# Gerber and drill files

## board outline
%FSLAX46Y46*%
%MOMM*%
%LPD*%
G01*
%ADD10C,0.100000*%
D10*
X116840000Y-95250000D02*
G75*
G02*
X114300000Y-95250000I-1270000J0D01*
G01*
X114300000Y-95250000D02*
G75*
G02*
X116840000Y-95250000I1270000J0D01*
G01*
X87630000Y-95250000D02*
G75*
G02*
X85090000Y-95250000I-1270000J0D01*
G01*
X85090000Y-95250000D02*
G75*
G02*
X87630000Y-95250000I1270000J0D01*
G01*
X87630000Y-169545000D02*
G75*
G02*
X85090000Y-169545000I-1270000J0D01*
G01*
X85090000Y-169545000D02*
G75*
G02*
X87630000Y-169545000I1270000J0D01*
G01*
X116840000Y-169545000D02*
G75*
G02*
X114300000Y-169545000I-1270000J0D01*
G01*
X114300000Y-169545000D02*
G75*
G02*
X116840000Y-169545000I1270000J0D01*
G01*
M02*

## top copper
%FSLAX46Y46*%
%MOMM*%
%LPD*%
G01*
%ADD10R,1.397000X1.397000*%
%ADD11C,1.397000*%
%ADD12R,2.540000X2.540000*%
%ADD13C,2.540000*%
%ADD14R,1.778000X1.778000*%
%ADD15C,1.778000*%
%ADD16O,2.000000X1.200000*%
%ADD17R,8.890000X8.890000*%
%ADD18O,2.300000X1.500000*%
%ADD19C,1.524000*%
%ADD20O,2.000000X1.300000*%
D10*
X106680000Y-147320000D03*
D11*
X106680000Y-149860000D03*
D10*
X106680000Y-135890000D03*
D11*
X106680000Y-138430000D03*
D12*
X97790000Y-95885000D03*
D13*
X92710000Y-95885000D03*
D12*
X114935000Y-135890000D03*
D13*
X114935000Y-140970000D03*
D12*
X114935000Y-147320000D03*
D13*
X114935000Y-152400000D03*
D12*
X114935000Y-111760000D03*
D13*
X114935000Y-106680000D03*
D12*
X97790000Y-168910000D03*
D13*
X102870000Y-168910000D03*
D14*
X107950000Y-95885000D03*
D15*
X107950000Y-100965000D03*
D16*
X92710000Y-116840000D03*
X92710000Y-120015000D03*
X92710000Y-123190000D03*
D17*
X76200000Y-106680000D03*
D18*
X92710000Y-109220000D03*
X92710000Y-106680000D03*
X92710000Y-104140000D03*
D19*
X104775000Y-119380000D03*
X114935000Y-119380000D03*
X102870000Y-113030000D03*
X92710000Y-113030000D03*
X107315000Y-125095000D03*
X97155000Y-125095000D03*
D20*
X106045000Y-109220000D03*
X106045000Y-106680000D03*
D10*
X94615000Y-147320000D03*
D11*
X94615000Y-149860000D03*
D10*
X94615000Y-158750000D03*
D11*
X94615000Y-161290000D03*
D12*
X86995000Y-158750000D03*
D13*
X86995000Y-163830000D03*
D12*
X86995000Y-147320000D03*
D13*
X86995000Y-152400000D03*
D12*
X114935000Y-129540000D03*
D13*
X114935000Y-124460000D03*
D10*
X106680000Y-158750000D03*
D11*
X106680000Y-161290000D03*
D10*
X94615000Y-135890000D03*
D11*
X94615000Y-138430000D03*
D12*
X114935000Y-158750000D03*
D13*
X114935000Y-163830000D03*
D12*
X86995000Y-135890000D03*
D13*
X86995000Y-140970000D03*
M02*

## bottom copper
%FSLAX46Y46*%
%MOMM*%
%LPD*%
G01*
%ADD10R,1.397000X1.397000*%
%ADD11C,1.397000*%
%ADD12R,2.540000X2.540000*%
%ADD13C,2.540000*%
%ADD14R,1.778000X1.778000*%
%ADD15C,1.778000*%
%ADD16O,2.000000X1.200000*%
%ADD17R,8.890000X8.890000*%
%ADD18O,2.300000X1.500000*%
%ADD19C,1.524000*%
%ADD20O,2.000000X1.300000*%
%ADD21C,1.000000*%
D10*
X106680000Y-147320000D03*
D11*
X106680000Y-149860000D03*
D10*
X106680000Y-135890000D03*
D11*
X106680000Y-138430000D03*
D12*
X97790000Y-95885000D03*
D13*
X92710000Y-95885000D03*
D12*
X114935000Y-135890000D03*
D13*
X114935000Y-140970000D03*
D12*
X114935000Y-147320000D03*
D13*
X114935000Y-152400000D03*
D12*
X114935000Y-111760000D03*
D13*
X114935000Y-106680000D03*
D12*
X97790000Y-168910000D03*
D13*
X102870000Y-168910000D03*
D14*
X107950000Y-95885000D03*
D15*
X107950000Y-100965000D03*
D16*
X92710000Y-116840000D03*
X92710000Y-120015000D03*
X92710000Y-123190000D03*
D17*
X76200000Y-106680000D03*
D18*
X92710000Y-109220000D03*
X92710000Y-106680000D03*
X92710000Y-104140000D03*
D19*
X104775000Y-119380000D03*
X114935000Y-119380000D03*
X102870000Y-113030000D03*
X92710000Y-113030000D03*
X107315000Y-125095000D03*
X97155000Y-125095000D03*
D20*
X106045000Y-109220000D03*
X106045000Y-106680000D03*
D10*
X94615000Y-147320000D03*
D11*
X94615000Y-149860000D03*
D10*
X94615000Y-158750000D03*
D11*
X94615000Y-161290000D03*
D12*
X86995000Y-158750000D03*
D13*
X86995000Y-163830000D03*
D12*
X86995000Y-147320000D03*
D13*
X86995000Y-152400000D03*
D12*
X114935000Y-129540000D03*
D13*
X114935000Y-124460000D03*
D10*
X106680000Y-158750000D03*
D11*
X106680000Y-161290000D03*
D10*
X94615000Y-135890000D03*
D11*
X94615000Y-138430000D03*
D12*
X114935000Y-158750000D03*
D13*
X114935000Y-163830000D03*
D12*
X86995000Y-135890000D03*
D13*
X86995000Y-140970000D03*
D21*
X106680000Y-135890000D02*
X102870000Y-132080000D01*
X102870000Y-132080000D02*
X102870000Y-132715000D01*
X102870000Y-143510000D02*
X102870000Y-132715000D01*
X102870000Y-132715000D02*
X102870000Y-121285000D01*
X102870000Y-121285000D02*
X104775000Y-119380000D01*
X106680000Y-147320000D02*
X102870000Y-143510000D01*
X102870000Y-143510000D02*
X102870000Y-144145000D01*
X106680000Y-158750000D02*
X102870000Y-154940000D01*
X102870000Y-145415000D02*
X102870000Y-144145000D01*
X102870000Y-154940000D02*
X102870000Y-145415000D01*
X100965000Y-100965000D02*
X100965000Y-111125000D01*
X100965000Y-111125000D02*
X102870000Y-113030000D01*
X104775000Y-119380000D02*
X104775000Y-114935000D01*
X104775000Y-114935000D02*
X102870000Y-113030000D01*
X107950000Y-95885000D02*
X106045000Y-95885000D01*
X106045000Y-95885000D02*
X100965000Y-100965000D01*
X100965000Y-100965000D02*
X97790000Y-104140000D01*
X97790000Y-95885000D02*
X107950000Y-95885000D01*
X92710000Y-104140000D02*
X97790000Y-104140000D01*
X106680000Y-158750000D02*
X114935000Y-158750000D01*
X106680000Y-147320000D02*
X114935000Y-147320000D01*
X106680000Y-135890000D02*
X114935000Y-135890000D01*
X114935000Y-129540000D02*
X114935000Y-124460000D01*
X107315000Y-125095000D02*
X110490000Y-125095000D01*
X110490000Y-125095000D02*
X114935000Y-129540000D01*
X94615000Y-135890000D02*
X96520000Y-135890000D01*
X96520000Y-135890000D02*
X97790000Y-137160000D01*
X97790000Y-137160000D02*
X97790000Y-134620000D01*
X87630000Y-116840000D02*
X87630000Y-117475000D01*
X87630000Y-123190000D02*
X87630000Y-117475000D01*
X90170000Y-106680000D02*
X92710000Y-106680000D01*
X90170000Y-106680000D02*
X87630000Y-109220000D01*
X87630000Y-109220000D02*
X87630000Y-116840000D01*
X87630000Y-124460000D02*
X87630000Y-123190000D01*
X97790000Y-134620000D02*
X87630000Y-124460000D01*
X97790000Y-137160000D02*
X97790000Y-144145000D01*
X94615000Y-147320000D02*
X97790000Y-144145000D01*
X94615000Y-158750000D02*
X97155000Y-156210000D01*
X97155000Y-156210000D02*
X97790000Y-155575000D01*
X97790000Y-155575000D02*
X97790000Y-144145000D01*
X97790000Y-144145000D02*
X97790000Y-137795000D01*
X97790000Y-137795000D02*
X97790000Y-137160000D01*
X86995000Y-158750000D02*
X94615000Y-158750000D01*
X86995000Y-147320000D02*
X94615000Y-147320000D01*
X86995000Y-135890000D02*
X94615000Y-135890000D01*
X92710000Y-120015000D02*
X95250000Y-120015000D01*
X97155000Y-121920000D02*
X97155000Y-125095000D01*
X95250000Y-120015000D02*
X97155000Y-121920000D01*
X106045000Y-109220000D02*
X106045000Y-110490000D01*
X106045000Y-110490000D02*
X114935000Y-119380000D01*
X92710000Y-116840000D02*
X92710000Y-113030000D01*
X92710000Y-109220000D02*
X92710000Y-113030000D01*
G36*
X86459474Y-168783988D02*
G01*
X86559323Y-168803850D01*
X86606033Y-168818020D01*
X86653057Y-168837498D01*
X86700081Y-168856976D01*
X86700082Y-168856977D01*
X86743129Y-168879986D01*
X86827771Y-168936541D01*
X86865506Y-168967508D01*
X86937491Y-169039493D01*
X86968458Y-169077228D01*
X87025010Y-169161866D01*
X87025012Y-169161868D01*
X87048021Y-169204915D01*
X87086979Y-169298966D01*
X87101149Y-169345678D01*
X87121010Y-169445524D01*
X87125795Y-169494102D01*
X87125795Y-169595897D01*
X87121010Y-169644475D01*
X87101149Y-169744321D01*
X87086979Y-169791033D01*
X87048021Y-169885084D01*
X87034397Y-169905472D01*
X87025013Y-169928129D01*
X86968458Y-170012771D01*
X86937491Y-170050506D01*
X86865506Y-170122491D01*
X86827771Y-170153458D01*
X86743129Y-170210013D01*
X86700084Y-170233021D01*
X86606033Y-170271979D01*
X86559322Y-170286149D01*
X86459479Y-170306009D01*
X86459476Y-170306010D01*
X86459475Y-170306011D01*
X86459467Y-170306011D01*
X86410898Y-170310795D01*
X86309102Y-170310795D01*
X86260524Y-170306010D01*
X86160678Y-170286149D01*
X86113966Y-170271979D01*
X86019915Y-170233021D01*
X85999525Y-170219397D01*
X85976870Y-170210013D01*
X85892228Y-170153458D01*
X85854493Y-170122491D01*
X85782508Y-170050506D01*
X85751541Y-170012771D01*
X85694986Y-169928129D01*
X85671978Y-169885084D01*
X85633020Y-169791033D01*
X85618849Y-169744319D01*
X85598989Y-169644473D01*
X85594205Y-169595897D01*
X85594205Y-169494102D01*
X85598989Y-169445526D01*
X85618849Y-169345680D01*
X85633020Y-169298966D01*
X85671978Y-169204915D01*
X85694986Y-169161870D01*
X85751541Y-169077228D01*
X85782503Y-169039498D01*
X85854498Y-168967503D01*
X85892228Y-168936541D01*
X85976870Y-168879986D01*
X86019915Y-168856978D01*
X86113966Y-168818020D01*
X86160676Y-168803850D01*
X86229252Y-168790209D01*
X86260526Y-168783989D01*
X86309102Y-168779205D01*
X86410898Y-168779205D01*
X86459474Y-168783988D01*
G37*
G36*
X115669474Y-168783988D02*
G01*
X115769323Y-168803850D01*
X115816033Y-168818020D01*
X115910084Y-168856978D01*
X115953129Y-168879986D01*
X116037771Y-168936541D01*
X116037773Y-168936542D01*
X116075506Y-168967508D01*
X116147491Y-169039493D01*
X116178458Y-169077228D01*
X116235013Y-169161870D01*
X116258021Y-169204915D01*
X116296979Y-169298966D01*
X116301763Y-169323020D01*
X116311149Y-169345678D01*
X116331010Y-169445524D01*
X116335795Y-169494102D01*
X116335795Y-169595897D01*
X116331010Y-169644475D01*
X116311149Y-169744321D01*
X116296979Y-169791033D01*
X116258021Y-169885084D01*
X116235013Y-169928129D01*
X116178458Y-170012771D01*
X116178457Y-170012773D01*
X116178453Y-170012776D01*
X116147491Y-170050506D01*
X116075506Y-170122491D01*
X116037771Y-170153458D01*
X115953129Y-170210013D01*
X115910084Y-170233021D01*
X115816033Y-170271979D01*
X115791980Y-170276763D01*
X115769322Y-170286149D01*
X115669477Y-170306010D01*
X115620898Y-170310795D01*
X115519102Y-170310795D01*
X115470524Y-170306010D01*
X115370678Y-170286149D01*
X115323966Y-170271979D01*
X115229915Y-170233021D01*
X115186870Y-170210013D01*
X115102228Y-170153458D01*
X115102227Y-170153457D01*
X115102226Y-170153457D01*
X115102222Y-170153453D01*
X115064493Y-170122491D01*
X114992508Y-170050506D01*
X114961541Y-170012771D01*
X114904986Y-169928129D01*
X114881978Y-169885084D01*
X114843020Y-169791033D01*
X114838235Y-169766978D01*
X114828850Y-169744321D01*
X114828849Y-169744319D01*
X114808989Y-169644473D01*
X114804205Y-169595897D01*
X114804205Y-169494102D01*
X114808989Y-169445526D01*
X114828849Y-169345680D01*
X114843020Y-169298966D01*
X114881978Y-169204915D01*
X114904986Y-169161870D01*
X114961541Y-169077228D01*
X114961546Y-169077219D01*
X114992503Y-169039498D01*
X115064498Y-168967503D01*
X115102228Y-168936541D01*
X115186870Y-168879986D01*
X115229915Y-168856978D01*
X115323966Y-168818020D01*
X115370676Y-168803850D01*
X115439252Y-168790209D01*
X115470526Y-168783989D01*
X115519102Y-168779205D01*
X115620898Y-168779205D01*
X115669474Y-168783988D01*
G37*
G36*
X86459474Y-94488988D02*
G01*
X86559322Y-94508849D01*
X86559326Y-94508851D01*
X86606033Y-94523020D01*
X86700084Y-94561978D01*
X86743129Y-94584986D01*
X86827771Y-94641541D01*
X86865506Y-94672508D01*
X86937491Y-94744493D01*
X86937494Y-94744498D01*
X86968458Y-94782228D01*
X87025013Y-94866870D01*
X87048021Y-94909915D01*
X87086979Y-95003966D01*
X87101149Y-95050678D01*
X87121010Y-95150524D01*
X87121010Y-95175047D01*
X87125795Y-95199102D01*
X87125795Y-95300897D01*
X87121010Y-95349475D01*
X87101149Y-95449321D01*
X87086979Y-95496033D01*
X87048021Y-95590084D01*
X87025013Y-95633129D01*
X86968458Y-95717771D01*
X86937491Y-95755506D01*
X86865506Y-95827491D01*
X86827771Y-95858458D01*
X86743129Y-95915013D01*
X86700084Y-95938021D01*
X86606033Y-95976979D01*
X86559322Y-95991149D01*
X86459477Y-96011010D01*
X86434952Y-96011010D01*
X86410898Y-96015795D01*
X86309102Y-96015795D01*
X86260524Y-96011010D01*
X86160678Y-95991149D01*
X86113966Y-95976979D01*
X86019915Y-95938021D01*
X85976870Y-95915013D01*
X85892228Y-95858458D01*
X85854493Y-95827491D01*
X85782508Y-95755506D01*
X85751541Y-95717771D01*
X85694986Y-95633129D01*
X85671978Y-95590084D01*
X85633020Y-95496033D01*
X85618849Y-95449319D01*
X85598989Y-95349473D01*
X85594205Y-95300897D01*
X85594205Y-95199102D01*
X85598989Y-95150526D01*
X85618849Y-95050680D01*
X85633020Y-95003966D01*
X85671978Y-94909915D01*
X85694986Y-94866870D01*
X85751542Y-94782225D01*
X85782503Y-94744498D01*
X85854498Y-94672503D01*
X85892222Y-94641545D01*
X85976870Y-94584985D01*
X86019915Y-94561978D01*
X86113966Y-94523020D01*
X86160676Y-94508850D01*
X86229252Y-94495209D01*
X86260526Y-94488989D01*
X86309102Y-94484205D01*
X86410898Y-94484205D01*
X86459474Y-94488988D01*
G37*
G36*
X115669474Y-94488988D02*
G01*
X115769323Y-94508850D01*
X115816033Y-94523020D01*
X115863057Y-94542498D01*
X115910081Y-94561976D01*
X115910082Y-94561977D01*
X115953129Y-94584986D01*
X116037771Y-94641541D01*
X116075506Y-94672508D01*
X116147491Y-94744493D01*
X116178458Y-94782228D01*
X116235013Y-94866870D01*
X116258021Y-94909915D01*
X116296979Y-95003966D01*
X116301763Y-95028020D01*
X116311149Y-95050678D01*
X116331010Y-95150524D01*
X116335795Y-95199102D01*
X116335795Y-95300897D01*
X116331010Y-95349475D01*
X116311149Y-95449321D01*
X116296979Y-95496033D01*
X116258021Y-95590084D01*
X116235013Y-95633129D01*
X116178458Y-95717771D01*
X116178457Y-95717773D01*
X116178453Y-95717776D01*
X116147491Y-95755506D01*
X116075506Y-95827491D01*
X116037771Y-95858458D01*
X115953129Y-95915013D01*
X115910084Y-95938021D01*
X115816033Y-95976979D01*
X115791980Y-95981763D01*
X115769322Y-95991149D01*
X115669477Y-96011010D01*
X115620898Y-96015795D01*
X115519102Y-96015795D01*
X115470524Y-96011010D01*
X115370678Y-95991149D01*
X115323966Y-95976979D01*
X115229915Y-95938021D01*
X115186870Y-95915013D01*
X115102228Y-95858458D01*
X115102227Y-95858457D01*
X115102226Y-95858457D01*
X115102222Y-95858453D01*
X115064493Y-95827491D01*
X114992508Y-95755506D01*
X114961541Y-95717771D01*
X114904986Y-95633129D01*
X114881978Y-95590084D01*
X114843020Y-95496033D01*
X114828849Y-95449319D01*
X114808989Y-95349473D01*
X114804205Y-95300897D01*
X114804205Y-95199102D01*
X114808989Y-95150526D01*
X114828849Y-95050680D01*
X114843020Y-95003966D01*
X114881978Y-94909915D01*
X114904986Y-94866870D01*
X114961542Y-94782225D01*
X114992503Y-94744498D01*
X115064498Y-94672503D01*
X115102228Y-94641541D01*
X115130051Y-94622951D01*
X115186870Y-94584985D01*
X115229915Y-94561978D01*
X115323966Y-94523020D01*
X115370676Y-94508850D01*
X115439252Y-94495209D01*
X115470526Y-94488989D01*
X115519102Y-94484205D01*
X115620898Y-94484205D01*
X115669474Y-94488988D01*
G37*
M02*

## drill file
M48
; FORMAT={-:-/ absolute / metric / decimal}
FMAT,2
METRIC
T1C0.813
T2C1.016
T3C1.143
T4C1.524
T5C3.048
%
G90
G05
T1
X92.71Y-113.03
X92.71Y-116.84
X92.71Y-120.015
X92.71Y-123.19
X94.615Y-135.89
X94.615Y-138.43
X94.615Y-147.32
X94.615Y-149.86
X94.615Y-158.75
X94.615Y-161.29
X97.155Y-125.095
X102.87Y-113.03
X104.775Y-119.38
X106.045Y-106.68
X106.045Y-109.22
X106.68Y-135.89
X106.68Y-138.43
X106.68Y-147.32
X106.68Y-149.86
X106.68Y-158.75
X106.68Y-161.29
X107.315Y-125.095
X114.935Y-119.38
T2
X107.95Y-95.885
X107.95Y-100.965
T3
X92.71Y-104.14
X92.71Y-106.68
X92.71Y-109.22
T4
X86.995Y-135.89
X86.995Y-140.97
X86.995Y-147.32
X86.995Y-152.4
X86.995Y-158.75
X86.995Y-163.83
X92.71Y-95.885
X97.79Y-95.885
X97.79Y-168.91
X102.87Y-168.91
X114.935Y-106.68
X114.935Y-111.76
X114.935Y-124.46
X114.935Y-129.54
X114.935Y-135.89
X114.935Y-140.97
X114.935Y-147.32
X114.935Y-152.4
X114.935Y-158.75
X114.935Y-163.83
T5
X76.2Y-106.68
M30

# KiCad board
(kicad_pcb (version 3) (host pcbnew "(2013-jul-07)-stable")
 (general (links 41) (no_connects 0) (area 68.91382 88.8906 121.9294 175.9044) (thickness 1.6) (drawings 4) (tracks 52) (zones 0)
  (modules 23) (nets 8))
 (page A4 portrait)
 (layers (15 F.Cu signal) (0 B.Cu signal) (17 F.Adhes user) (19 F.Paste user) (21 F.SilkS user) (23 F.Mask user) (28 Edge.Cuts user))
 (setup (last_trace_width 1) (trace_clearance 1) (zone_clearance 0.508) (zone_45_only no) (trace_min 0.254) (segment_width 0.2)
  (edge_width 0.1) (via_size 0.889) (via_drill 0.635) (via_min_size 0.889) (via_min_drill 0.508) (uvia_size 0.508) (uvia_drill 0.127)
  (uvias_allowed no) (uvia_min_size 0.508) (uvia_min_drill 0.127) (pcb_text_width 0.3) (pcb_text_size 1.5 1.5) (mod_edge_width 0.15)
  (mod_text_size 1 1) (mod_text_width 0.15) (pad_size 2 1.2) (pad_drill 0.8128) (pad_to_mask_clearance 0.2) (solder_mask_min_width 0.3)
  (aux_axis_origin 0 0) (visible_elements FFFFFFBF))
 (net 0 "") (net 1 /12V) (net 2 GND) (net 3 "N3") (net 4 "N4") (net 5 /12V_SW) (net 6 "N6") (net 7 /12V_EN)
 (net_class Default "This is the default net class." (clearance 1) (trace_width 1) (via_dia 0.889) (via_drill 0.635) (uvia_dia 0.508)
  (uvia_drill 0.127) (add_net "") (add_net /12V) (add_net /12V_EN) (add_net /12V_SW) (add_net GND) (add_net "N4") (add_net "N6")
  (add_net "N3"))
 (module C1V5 (layer F.Cu) (at 106.68 148.59 270)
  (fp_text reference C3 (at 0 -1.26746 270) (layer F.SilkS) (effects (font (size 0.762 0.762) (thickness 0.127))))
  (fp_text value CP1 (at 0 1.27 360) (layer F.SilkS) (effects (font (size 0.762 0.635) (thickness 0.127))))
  (pad 1 thru_hole rect (at -1.27 0 270) (size 1.397 1.397) (drill 0.8128) (layers *.Cu *.Mask F.SilkS) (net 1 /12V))
  (pad 2 thru_hole circle (at 1.27 0 270) (size 1.397 1.397) (drill 0.8128) (layers *.Cu *.Mask F.SilkS) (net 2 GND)))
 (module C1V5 (layer F.Cu) (at 106.68 137.16 270)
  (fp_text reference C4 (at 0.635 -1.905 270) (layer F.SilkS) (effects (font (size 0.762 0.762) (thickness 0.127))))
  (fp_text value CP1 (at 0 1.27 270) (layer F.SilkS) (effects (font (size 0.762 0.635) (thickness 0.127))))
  (pad 1 thru_hole rect (at -1.27 0 270) (size 1.397 1.397) (drill 0.8128) (layers *.Cu *.Mask F.SilkS) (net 1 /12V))
  (pad 2 thru_hole circle (at 1.27 0 270) (size 1.397 1.397) (drill 0.8128) (layers *.Cu *.Mask F.SilkS) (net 2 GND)))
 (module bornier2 (layer F.Cu) (at 95.25 95.885 180)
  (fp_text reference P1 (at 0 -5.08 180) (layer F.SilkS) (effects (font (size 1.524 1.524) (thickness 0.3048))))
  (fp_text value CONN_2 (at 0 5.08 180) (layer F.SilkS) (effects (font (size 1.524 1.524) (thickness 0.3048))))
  (pad 1 thru_hole rect (at -2.54 0 180) (size 2.54 2.54) (drill 1.524) (layers *.Cu *.Mask F.SilkS) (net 1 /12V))
  (pad 2 thru_hole circle (at 2.54 0 180) (size 2.54 2.54) (drill 1.524) (layers *.Cu *.Mask F.SilkS) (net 2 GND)))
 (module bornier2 (layer F.Cu) (at 114.935 138.43 270)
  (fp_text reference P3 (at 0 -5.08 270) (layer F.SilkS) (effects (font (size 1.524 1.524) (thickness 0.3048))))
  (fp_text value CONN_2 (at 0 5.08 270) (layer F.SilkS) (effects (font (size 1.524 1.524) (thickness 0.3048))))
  (pad 1 thru_hole rect (at -2.54 0 270) (size 2.54 2.54) (drill 1.524) (layers *.Cu *.Mask F.SilkS) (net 1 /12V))
  (pad 2 thru_hole circle (at 2.54 0 270) (size 2.54 2.54) (drill 1.524) (layers *.Cu *.Mask F.SilkS) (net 2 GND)))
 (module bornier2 (layer F.Cu) (at 114.935 149.86 270)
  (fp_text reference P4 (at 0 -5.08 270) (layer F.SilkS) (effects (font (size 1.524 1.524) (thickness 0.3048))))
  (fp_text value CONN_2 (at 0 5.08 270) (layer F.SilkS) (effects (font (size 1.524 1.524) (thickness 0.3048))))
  (pad 1 thru_hole rect (at -2.54 0 270) (size 2.54 2.54) (drill 1.524) (layers *.Cu *.Mask F.SilkS) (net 1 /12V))
  (pad 2 thru_hole circle (at 2.54 0 270) (size 2.54 2.54) (drill 1.524) (layers *.Cu *.Mask F.SilkS) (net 2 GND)))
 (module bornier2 (layer F.Cu) (at 114.935 109.22 90)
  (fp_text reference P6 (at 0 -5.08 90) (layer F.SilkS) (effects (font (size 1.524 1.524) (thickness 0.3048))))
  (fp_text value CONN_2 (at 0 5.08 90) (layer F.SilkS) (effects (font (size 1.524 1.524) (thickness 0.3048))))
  (pad 1 thru_hole rect (at -2.54 0 90) (size 2.54 2.54) (drill 1.524) (layers *.Cu *.Mask F.SilkS) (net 2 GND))
  (pad 2 thru_hole circle (at 2.54 0 90) (size 2.54 2.54) (drill 1.524) (layers *.Cu *.Mask F.SilkS) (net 2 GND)))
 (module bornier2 (layer F.Cu) (at 100.33 168.91)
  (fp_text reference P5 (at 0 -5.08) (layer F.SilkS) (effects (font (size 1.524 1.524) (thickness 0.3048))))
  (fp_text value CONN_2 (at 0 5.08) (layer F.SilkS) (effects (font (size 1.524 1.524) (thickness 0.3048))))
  (pad 1 thru_hole rect (at -2.54 0) (size 2.54 2.54) (drill 1.524) (layers *.Cu *.Mask F.SilkS) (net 2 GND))
  (pad 2 thru_hole circle (at 2.54 0) (size 2.54 2.54) (drill 1.524) (layers *.Cu *.Mask F.SilkS) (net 2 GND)))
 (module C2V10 (layer F.Cu) (at 107.95 98.425 270)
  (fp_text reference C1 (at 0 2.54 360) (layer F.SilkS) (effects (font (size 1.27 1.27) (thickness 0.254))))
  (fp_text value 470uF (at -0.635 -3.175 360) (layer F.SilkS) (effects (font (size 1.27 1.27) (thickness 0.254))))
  (pad 1 thru_hole rect (at -2.54 0 270) (size 1.778 1.778) (drill 1.016) (layers *.Cu *.Mask F.SilkS) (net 1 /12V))
  (pad 2 thru_hole circle (at 2.54 0 270) (size 1.778 1.778) (drill 1.016) (layers *.Cu *.Mask F.SilkS) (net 2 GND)))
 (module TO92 (layer F.Cu) (at 92.71 120.015 45)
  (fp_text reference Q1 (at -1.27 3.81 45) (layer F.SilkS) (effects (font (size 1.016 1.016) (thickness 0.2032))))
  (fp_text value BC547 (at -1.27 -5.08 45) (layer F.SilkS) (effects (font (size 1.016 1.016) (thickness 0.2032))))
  (pad 1 thru_hole oval (at 2.245064 -2.245064 180) (size 2 1.2) (drill 0.8128) (layers *.Cu *.Mask F.SilkS) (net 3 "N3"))
  (pad 2 thru_hole oval (at 0 0 180) (size 2 1.2) (drill 0.8128) (layers *.Cu *.Mask F.SilkS) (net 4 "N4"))
  (pad 3 thru_hole oval (at -2.245064 2.245064 180) (size 2 1.2) (drill 0.8128) (layers *.Cu *.Mask F.SilkS) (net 2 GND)))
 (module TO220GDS (layer F.Cu) (at 92.71 106.68 180)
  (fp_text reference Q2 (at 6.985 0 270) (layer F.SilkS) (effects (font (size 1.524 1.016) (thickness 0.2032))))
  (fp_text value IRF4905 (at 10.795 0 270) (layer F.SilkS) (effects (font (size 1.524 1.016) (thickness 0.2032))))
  (pad 4 thru_hole rect (at 16.51 0 180) (size 8.89 8.89) (drill 3.048) (layers *.Cu *.SilkS *.Mask))
  (pad G thru_hole oval (at 0 -2.54 180) (size 2.3 1.5) (drill 1.143) (layers *.Cu *.Mask F.SilkS) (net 3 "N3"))
  (pad D thru_hole oval (at 0 0 180) (size 2.3 1.5) (drill 1.143) (layers *.Cu *.Mask F.SilkS) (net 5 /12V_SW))
  (pad S thru_hole oval (at 0 2.54 180) (size 2.3 1.5) (drill 1.143) (layers *.Cu *.Mask F.SilkS) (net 1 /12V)))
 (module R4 (layer F.Cu) (at 109.855 119.38) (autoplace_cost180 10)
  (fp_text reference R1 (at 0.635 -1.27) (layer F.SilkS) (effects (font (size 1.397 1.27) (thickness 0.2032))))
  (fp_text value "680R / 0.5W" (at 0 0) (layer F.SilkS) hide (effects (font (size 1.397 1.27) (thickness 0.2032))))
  (pad 1 thru_hole circle (at -5.08 0) (size 1.524 1.524) (drill 0.8128) (layers *.Cu *.Mask F.SilkS) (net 1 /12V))
  (pad 2 thru_hole circle (at 5.08 0) (size 1.524 1.524) (drill 0.8128) (layers *.Cu *.Mask F.SilkS) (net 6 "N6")))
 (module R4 (layer F.Cu) (at 97.79 113.03 180) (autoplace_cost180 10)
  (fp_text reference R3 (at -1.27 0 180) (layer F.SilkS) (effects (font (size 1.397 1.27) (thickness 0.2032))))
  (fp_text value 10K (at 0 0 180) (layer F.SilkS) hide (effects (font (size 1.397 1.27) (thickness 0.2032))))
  (pad 1 thru_hole circle (at -5.08 0 180) (size 1.524 1.524) (drill 0.8128) (layers *.Cu *.Mask F.SilkS) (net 1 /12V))
  (pad 2 thru_hole circle (at 5.08 0 180) (size 1.524 1.524) (drill 0.8128) (layers *.Cu *.Mask F.SilkS) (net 3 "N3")))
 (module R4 (layer F.Cu) (at 102.235 125.095 180) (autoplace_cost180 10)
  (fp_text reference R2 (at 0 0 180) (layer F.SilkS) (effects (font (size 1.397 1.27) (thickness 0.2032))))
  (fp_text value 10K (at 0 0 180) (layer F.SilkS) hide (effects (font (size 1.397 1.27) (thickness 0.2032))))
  (pad 1 thru_hole circle (at -5.08 0 180) (size 1.524 1.524) (drill 0.8128) (layers *.Cu *.Mask F.SilkS) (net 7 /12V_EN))
  (pad 2 thru_hole circle (at 5.08 0 180) (size 1.524 1.524) (drill 0.8128) (layers *.Cu *.Mask F.SilkS) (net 4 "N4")))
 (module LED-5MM (layer F.Cu) (at 106.045 107.95 90)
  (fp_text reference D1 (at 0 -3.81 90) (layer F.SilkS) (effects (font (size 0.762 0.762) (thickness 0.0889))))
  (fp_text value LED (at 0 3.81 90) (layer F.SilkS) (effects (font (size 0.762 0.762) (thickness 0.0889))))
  (pad 1 thru_hole oval (at -1.27 0 90) (size 1.3 2) (drill 0.8128) (layers *.Cu *.Mask F.SilkS) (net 6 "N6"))
  (pad 2 thru_hole oval (at 1.27 0 90) (size 1.3 2) (drill 0.8128) (layers *.Cu *.Mask F.SilkS) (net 2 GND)))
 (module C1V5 (layer F.Cu) (at 94.615 148.59 270)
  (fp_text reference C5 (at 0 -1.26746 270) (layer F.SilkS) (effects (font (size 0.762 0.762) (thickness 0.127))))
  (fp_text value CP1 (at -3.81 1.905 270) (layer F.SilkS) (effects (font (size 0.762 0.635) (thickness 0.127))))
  (pad 1 thru_hole rect (at -1.27 0 270) (size 1.397 1.397) (drill 0.8128) (layers *.Cu *.Mask F.SilkS) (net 5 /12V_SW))
  (pad 2 thru_hole circle (at 1.27 0 270) (size 1.397 1.397) (drill 0.8128) (layers *.Cu *.Mask F.SilkS) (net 2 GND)))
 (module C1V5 (layer F.Cu) (at 94.615 160.02 270)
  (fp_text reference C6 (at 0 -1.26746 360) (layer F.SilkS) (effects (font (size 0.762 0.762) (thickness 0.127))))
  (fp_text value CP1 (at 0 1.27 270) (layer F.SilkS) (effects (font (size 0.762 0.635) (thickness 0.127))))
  (pad 1 thru_hole rect (at -1.27 0 270) (size 1.397 1.397) (drill 0.8128) (layers *.Cu *.Mask F.SilkS) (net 5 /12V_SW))
  (pad 2 thru_hole circle (at 1.27 0 270) (size 1.397 1.397) (drill 0.8128) (layers *.Cu *.Mask F.SilkS) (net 2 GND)))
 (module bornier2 (layer F.Cu) (at 86.995 161.29 270)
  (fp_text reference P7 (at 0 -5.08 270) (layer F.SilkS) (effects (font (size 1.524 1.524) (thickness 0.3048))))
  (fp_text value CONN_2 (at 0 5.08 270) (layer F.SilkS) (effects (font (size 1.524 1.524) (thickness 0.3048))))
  (pad 1 thru_hole rect (at -2.54 0 270) (size 2.54 2.54) (drill 1.524) (layers *.Cu *.Mask F.SilkS) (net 5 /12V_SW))
  (pad 2 thru_hole circle (at 2.54 0 270) (size 2.54 2.54) (drill 1.524) (layers *.Cu *.Mask F.SilkS) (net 2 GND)))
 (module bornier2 (layer F.Cu) (at 86.995 149.86 270)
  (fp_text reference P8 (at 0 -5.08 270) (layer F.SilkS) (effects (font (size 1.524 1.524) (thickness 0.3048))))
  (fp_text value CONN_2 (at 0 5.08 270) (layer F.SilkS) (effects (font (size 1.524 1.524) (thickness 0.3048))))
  (pad 1 thru_hole rect (at -2.54 0 270) (size 2.54 2.54) (drill 1.524) (layers *.Cu *.Mask F.SilkS) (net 5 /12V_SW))
  (pad 2 thru_hole circle (at 2.54 0 270) (size 2.54 2.54) (drill 1.524) (layers *.Cu *.Mask F.SilkS) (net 2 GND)))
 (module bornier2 (layer F.Cu) (at 114.935 127 90)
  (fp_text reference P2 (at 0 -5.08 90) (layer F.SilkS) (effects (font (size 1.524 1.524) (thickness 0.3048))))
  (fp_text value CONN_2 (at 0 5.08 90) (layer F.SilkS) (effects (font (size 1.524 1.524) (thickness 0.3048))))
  (pad 1 thru_hole rect (at -2.54 0 90) (size 2.54 2.54) (drill 1.524) (layers *.Cu *.Mask F.SilkS) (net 7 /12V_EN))
  (pad 2 thru_hole circle (at 2.54 0 90) (size 2.54 2.54) (drill 1.524) (layers *.Cu *.Mask F.SilkS) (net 7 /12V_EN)))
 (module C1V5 (layer F.Cu) (at 106.68 160.02 270)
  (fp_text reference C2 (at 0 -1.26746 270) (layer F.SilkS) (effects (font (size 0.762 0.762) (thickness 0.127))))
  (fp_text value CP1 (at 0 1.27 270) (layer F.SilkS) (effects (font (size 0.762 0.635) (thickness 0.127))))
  (pad 1 thru_hole rect (at -1.27 0 270) (size 1.397 1.397) (drill 0.8128) (layers *.Cu *.Mask F.SilkS) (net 1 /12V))
  (pad 2 thru_hole circle (at 1.27 0 270) (size 1.397 1.397) (drill 0.8128) (layers *.Cu *.Mask F.SilkS) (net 2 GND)))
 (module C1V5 (layer F.Cu) (at 94.615 137.16 270)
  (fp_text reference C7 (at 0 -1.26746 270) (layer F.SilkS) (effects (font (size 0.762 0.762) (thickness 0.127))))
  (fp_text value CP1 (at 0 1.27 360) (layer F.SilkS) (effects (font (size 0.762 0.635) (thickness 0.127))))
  (pad 1 thru_hole rect (at -1.27 0 270) (size 1.397 1.397) (drill 0.8128) (layers *.Cu *.Mask F.SilkS) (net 5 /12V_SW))
  (pad 2 thru_hole circle (at 1.27 0 270) (size 1.397 1.397) (drill 0.8128) (layers *.Cu *.Mask F.SilkS) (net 2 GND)))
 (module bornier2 (layer F.Cu) (at 114.935 161.29 270)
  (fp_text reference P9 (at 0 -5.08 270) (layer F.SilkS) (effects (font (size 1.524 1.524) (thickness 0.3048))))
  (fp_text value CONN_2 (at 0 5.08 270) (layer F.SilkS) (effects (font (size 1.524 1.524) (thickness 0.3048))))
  (pad 1 thru_hole rect (at -2.54 0 270) (size 2.54 2.54) (drill 1.524) (layers *.Cu *.Mask F.SilkS) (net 1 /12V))
  (pad 2 thru_hole circle (at 2.54 0 270) (size 2.54 2.54) (drill 1.524) (layers *.Cu *.Mask F.SilkS) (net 2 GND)))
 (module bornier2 (layer F.Cu) (at 86.995 138.43 270)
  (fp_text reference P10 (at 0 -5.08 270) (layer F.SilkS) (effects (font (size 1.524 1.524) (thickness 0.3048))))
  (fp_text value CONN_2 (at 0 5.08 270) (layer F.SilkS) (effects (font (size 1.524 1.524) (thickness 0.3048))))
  (pad 1 thru_hole rect (at -2.54 0 270) (size 2.54 2.54) (drill 1.524) (layers *.Cu *.Mask F.SilkS) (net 5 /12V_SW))
  (pad 2 thru_hole circle (at 2.54 0 270) (size 2.54 2.54) (drill 1.524) (layers *.Cu *.Mask F.SilkS) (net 2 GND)))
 (gr_circle (center 115.57 95.25) (end 116.84 95.25) (layer Edge.Cuts) (width 0.1))
 (gr_circle (center 86.36 95.25) (end 87.63 95.25) (layer Edge.Cuts) (width 0.1))
 (gr_circle (center 86.36 169.545) (end 87.63 169.545) (layer Edge.Cuts) (width 0.1))
 (gr_circle (center 115.57 169.545) (end 114.3 169.545) (layer Edge.Cuts) (width 0.1))
 (segment (start 106.68 135.89) (end 102.87 132.08) (width 1) (layer B.Cu) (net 1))
 (segment (start 102.87 132.08) (end 102.87 132.715) (width 1) (layer B.Cu) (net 1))
 (segment (start 102.87 143.51) (end 102.87 132.715) (width 1) (layer B.Cu) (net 1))
 (segment (start 102.87 132.715) (end 102.87 121.285) (width 1) (layer B.Cu) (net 1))
 (segment (start 102.87 121.285) (end 104.775 119.38) (width 1) (layer B.Cu) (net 1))
 (segment (start 106.68 147.32) (end 102.87 143.51) (width 1) (layer B.Cu) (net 1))
 (segment (start 102.87 143.51) (end 102.87 144.145) (width 1) (layer B.Cu) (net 1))
 (segment (start 106.68 158.75) (end 102.87 154.94) (width 1) (layer B.Cu) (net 1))
 (segment (start 102.87 145.415) (end 102.87 144.145) (width 1) (layer B.Cu) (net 1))
 (segment (start 102.87 154.94) (end 102.87 145.415) (width 1) (layer B.Cu) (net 1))
 (segment (start 100.965 100.965) (end 100.965 111.125) (width 1) (layer B.Cu) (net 1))
 (segment (start 100.965 111.125) (end 102.87 113.03) (width 1) (layer B.Cu) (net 1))
 (segment (start 104.775 119.38) (end 104.775 114.935) (width 1) (layer B.Cu) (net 1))
 (segment (start 104.775 114.935) (end 102.87 113.03) (width 1) (layer B.Cu) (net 1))
 (segment (start 107.95 95.885) (end 106.045 95.885) (width 1) (layer B.Cu) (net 1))
 (segment (start 106.045 95.885) (end 100.965 100.965) (width 1) (layer B.Cu) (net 1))
 (segment (start 100.965 100.965) (end 97.79 104.14) (width 1) (layer B.Cu) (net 1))
 (segment (start 97.79 95.885) (end 107.95 95.885) (width 1) (layer B.Cu) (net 1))
 (segment (start 92.71 104.14) (end 97.79 104.14) (width 1) (layer B.Cu) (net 1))
 (segment (start 106.68 158.75) (end 114.935 158.75) (width 1) (layer B.Cu) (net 1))
 (segment (start 106.68 147.32) (end 114.935 147.32) (width 1) (layer B.Cu) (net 1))
 (segment (start 106.68 135.89) (end 114.935 135.89) (width 1) (layer B.Cu) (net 1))
 (segment (start 114.935 129.54) (end 114.935 124.46) (width 1) (layer B.Cu) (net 7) (status C00000))
 (segment (start 107.315 125.095) (end 110.49 125.095) (width 1) (layer B.Cu) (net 7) (status 400000))
 (segment (start 110.49 125.095) (end 114.935 129.54) (width 1) (layer B.Cu) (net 7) (status 800000))
 (segment (start 94.615 135.89) (end 96.52 135.89) (width 1) (layer B.Cu) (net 5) (status 400000))
 (segment (start 96.52 135.89) (end 97.79 137.16) (width 1) (layer B.Cu) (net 5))
 (segment (start 97.79 137.16) (end 97.79 134.62) (width 1) (layer B.Cu) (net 5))
 (segment (start 87.63 116.84) (end 87.63 117.475) (width 1) (layer B.Cu) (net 5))
 (segment (start 87.63 123.19) (end 87.63 117.475) (width 1) (layer B.Cu) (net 5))
 (segment (start 90.17 106.68) (end 92.71 106.68) (width 1) (layer B.Cu) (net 5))
 (segment (start 90.17 106.68) (end 87.63 109.22) (width 1) (layer B.Cu) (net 5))
 (segment (start 87.63 109.22) (end 87.63 116.84) (width 1) (layer B.Cu) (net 5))
 (segment (start 87.63 124.46) (end 87.63 123.19) (width 1) (layer B.Cu) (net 5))
 (segment (start 97.79 134.62) (end 87.63 124.46) (width 1) (layer B.Cu) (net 5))
 (segment (start 97.79 137.16) (end 97.79 144.145) (width 1) (layer B.Cu) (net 5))
 (segment (start 94.615 147.32) (end 97.79 144.145) (width 1) (layer B.Cu) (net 5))
 (segment (start 94.615 158.75) (end 97.155 156.21) (width 1) (layer B.Cu) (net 5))
 (segment (start 97.155 156.21) (end 97.79 155.575) (width 1) (layer B.Cu) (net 5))
 (segment (start 97.79 155.575) (end 97.79 144.145) (width 1) (layer B.Cu) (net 5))
 (segment (start 97.79 144.145) (end 97.79 137.795) (width 1) (layer B.Cu) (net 5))
 (segment (start 97.79 137.795) (end 97.79 137.16) (width 1) (layer B.Cu) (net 5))
 (segment (start 86.995 158.75) (end 94.615 158.75) (width 1) (layer B.Cu) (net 5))
 (segment (start 86.995 147.32) (end 94.615 147.32) (width 1) (layer B.Cu) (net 5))
 (segment (start 86.995 135.89) (end 94.615 135.89) (width 1) (layer B.Cu) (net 5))
 (segment (start 92.71 120.015) (end 95.25 120.015) (width 1) (layer B.Cu) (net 4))
 (segment (start 97.155 121.92) (end 97.155 125.095) (width 1) (layer B.Cu) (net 4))
 (segment (start 95.25 120.015) (end 97.155 121.92) (width 1) (layer B.Cu) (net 4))
 (segment (start 106.045 109.22) (end 106.045 110.49) (width 1) (layer B.Cu) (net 6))
 (segment (start 106.045 110.49) (end 114.935 119.38) (width 1) (layer B.Cu) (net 6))
 (segment (start 92.71 116.84) (end 92.71 113.03) (width 1) (layer B.Cu) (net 3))
 (segment (start 92.71 109.22) (end 92.71 113.03) (width 1) (layer B.Cu) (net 3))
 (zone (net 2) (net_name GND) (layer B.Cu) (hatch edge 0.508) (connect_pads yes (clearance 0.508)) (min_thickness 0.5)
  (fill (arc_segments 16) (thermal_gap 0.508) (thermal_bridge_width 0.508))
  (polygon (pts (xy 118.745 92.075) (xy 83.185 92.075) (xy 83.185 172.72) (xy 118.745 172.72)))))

